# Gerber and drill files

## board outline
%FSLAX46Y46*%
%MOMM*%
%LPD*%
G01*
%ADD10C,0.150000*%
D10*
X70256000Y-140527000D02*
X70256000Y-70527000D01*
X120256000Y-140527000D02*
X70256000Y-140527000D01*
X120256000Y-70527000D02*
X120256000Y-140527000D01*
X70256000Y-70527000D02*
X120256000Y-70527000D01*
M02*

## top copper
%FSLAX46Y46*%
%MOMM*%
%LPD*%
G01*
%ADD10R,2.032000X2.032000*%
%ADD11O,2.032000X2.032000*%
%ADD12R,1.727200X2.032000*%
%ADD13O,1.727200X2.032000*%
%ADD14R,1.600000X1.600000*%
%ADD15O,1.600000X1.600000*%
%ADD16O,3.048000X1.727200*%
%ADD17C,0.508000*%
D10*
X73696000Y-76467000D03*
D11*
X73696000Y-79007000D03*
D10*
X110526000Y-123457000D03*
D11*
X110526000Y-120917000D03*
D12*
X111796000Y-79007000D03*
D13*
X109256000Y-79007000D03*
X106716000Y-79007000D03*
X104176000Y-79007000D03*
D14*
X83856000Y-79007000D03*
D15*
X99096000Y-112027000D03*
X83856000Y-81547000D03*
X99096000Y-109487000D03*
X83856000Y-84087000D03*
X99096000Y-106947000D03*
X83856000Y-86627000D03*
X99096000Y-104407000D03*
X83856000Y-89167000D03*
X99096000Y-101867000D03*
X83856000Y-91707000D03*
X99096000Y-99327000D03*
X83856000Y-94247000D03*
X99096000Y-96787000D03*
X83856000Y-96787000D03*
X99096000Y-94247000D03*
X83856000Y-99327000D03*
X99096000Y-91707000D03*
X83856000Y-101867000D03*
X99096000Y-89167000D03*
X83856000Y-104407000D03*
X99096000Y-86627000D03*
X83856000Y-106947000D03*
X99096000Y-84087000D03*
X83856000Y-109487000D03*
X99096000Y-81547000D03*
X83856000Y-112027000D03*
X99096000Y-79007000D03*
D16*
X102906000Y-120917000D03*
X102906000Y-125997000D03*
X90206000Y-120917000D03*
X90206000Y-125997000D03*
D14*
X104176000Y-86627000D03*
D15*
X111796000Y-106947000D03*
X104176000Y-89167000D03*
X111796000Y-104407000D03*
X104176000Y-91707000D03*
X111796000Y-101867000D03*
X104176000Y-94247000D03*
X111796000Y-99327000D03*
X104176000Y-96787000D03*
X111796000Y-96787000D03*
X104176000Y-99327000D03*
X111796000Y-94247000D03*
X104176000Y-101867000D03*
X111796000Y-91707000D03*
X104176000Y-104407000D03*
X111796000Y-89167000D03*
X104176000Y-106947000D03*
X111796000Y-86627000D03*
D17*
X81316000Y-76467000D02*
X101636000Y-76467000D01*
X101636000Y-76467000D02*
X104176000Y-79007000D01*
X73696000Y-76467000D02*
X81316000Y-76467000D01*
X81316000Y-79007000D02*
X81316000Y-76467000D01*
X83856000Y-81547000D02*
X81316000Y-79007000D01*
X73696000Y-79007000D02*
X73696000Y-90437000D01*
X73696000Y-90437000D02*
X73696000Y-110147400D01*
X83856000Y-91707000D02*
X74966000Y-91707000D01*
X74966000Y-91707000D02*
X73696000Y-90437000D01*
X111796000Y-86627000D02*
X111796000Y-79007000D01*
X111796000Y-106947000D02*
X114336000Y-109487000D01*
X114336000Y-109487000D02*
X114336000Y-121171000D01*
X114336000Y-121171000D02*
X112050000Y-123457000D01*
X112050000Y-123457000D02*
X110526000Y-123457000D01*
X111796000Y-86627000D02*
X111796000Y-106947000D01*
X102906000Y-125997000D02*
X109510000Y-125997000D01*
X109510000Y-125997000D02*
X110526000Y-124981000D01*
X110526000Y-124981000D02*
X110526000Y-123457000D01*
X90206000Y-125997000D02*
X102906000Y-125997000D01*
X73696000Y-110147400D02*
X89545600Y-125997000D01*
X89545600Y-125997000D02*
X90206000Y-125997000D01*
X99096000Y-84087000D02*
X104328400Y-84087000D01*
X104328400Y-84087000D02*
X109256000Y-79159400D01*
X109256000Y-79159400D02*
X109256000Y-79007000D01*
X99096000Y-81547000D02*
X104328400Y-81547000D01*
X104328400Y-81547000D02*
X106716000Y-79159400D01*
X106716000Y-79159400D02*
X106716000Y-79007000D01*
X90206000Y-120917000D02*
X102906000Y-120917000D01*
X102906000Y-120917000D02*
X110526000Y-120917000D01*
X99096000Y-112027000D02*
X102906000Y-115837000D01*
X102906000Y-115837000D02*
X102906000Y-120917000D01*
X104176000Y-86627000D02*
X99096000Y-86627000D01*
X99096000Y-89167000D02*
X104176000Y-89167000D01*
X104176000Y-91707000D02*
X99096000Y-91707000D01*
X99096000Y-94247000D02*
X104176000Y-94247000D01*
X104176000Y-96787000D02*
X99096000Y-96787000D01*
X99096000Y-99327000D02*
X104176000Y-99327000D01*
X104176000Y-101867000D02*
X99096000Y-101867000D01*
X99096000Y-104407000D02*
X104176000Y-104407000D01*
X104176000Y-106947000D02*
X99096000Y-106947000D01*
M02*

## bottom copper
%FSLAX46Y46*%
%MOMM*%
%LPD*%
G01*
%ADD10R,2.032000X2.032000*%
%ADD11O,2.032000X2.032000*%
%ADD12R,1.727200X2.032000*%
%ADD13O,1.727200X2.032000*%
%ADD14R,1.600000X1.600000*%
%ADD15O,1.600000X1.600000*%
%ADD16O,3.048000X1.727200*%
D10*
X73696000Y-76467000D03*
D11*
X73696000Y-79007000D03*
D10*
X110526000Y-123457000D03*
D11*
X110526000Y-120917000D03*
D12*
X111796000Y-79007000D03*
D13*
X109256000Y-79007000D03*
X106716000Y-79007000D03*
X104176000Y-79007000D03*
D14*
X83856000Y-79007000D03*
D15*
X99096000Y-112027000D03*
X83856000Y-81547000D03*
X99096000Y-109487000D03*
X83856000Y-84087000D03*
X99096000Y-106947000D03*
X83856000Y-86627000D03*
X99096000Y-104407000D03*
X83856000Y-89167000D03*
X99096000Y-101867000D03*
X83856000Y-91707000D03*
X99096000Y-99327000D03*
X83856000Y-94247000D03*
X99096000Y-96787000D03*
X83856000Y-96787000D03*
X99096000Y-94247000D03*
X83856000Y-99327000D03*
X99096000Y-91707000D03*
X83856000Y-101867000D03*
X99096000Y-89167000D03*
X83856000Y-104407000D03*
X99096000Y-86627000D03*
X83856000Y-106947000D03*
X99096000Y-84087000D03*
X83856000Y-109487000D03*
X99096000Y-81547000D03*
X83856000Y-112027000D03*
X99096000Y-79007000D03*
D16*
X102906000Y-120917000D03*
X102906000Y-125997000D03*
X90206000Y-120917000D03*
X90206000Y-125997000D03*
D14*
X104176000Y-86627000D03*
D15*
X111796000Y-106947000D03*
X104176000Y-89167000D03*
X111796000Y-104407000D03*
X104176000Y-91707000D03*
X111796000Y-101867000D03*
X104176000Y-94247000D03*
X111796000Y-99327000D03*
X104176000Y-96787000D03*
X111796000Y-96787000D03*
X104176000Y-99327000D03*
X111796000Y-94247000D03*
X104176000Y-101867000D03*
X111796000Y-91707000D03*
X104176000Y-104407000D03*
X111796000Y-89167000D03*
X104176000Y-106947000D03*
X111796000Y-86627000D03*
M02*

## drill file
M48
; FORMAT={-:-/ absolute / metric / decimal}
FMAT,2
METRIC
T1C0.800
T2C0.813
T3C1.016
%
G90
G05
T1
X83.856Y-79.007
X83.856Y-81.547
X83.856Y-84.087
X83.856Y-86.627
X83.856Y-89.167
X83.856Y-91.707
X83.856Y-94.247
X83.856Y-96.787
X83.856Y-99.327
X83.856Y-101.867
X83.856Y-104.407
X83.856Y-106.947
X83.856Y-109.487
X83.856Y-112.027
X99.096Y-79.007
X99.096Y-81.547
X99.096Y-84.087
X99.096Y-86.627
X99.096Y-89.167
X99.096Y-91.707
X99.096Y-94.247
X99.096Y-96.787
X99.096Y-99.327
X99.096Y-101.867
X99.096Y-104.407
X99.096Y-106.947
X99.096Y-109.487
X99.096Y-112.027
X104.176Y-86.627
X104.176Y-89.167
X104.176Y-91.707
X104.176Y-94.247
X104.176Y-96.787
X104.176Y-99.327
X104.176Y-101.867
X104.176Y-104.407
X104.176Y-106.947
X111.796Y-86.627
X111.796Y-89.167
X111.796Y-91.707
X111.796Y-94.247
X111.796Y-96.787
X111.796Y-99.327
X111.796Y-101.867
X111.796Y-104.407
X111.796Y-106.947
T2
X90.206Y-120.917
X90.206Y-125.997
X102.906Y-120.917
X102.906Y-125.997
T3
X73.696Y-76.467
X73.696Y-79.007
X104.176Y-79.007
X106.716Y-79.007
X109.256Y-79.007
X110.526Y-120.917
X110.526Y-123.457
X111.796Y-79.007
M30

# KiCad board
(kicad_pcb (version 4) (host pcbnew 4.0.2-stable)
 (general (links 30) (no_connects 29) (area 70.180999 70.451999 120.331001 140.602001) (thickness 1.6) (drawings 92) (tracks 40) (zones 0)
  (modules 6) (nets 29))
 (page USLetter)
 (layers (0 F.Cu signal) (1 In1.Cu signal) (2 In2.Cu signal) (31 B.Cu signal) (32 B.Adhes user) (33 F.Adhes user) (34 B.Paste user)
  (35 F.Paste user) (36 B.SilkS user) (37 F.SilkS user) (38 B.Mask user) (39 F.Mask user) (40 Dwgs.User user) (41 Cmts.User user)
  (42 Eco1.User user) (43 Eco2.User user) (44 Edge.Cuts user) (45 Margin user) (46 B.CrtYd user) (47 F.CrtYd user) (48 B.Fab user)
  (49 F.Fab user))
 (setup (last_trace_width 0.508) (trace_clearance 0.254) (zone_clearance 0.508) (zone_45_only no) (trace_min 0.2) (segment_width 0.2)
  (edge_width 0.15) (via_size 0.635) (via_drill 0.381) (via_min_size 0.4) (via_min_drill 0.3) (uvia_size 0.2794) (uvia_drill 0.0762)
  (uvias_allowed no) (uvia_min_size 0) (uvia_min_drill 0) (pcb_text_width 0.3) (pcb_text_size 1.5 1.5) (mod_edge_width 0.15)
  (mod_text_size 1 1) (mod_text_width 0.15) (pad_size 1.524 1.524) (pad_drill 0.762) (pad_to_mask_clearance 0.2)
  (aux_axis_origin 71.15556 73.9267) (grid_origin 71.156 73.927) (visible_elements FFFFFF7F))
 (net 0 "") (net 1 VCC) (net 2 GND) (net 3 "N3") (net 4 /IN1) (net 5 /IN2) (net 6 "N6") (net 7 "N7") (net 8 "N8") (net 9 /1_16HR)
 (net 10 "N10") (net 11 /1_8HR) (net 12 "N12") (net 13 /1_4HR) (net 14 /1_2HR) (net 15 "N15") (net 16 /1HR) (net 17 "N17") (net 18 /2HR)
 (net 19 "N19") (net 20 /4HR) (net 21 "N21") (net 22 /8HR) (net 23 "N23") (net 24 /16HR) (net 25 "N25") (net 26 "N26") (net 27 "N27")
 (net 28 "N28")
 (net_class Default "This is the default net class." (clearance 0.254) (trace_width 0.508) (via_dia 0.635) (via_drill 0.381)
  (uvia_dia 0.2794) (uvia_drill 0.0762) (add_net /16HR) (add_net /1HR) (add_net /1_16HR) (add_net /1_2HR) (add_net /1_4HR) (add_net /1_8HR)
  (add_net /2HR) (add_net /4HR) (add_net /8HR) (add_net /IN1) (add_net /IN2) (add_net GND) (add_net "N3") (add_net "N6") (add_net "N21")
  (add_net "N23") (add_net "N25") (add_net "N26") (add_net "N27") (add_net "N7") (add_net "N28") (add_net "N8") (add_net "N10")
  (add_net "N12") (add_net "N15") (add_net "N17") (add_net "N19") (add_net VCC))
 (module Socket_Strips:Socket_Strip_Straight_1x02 (layer F.Cu) (at 73.696 76.467 270)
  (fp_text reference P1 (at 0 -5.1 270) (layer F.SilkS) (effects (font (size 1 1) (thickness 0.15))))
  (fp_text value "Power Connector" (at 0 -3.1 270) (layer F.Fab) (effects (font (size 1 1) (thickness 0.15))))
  (pad 1 thru_hole rect (at 0 0 270) (size 2.032 2.032) (drill 1.016) (layers *.Cu *.Mask) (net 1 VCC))
  (pad 2 thru_hole oval (at 2.54 0 270) (size 2.032 2.032) (drill 1.016) (layers *.Cu *.Mask) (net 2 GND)))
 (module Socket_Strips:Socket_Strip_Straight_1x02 (layer F.Cu) (at 110.526 123.457 90)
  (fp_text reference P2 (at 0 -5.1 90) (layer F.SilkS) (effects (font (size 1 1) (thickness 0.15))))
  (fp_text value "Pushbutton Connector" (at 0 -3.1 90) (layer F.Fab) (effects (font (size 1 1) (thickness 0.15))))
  (pad 1 thru_hole rect (at 0 0 90) (size 2.032 2.032) (drill 1.016) (layers *.Cu *.Mask) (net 2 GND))
  (pad 2 thru_hole oval (at 2.54 0 90) (size 2.032 2.032) (drill 1.016) (layers *.Cu *.Mask) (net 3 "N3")))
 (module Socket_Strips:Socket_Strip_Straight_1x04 (layer F.Cu) (at 111.796 79.007 180)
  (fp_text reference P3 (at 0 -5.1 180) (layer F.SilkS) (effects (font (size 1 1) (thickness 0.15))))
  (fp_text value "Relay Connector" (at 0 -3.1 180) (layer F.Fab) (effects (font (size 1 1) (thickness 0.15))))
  (pad 1 thru_hole rect (at 0 0 180) (size 1.7272 2.032) (drill 1.016) (layers *.Cu *.Mask) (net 2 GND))
  (pad 2 thru_hole oval (at 2.54 0 180) (size 1.7272 2.032) (drill 1.016) (layers *.Cu *.Mask) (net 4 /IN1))
  (pad 3 thru_hole oval (at 5.08 0 180) (size 1.7272 2.032) (drill 1.016) (layers *.Cu *.Mask) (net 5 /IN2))
  (pad 4 thru_hole oval (at 7.62 0 180) (size 1.7272 2.032) (drill 1.016) (layers *.Cu *.Mask) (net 1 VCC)))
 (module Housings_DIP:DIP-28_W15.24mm (layer F.Cu) (at 83.856 79.007)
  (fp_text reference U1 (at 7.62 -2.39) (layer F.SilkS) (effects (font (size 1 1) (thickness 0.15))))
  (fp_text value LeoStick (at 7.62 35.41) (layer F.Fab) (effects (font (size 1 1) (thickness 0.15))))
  (pad 1 thru_hole rect (at 0 0) (size 1.6 1.6) (drill 0.8) (layers *.Cu *.Mask) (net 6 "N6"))
  (pad 15 thru_hole oval (at 15.24 33.02) (size 1.6 1.6) (drill 0.8) (layers *.Cu *.Mask) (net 3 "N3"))
  (pad 2 thru_hole oval (at 0 2.54) (size 1.6 1.6) (drill 0.8) (layers *.Cu *.Mask) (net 1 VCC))
  (pad 16 thru_hole oval (at 15.24 30.48) (size 1.6 1.6) (drill 0.8) (layers *.Cu *.Mask) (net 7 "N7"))
  (pad 3 thru_hole oval (at 0 5.08) (size 1.6 1.6) (drill 0.8) (layers *.Cu *.Mask) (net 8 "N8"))
  (pad 17 thru_hole oval (at 15.24 27.94) (size 1.6 1.6) (drill 0.8) (layers *.Cu *.Mask) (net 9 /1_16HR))
  (pad 4 thru_hole oval (at 0 7.62) (size 1.6 1.6) (drill 0.8) (layers *.Cu *.Mask) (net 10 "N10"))
  (pad 18 thru_hole oval (at 15.24 25.4) (size 1.6 1.6) (drill 0.8) (layers *.Cu *.Mask) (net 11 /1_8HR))
  (pad 5 thru_hole oval (at 0 10.16) (size 1.6 1.6) (drill 0.8) (layers *.Cu *.Mask) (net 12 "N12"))
  (pad 19 thru_hole oval (at 15.24 22.86) (size 1.6 1.6) (drill 0.8) (layers *.Cu *.Mask) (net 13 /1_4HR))
  (pad 6 thru_hole oval (at 0 12.7) (size 1.6 1.6) (drill 0.8) (layers *.Cu *.Mask) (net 2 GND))
  (pad 20 thru_hole oval (at 15.24 20.32) (size 1.6 1.6) (drill 0.8) (layers *.Cu *.Mask) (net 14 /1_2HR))
  (pad 7 thru_hole oval (at 0 15.24) (size 1.6 1.6) (drill 0.8) (layers *.Cu *.Mask) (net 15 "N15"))
  (pad 21 thru_hole oval (at 15.24 17.78) (size 1.6 1.6) (drill 0.8) (layers *.Cu *.Mask) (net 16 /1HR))
  (pad 8 thru_hole oval (at 0 17.78) (size 1.6 1.6) (drill 0.8) (layers *.Cu *.Mask) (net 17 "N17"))
  (pad 22 thru_hole oval (at 15.24 15.24) (size 1.6 1.6) (drill 0.8) (layers *.Cu *.Mask) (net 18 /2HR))
  (pad 9 thru_hole oval (at 0 20.32) (size 1.6 1.6) (drill 0.8) (layers *.Cu *.Mask) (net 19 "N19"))
  (pad 23 thru_hole oval (at 15.24 12.7) (size 1.6 1.6) (drill 0.8) (layers *.Cu *.Mask) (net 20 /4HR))
  (pad 10 thru_hole oval (at 0 22.86) (size 1.6 1.6) (drill 0.8) (layers *.Cu *.Mask) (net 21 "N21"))
  (pad 24 thru_hole oval (at 15.24 10.16) (size 1.6 1.6) (drill 0.8) (layers *.Cu *.Mask) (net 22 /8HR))
  (pad 11 thru_hole oval (at 0 25.4) (size 1.6 1.6) (drill 0.8) (layers *.Cu *.Mask) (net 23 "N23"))
  (pad 25 thru_hole oval (at 15.24 7.62) (size 1.6 1.6) (drill 0.8) (layers *.Cu *.Mask) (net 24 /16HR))
  (pad 12 thru_hole oval (at 0 27.94) (size 1.6 1.6) (drill 0.8) (layers *.Cu *.Mask) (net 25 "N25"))
  (pad 26 thru_hole oval (at 15.24 5.08) (size 1.6 1.6) (drill 0.8) (layers *.Cu *.Mask) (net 4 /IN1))
  (pad 13 thru_hole oval (at 0 30.48) (size 1.6 1.6) (drill 0.8) (layers *.Cu *.Mask) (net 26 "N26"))
  (pad 27 thru_hole oval (at 15.24 2.54) (size 1.6 1.6) (drill 0.8) (layers *.Cu *.Mask) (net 5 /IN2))
  (pad 14 thru_hole oval (at 0 33.02) (size 1.6 1.6) (drill 0.8) (layers *.Cu *.Mask) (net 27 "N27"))
  (pad 28 thru_hole oval (at 15.24 0) (size 1.6 1.6) (drill 0.8) (layers *.Cu *.Mask) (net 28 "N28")))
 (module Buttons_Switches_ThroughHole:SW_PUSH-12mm (layer F.Cu) (at 96.556 123.457)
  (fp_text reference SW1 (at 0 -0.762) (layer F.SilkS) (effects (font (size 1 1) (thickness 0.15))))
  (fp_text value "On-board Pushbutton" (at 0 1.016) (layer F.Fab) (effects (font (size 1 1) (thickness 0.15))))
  (pad 1 thru_hole oval (at 6.35 -2.54) (size 3.048 1.7272) (drill 0.8128) (layers *.Cu *.Mask) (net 3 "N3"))
  (pad 2 thru_hole oval (at 6.35 2.54) (size 3.048 1.7272) (drill 0.8128) (layers *.Cu *.Mask) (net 2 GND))
  (pad 1 thru_hole oval (at -6.35 -2.54) (size 3.048 1.7272) (drill 0.8128) (layers *.Cu *.Mask) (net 3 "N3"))
  (pad 2 thru_hole oval (at -6.35 2.54) (size 3.048 1.7272) (drill 0.8128) (layers *.Cu *.Mask) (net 2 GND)))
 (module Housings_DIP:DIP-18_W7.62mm (layer F.Cu) (at 104.176 86.627)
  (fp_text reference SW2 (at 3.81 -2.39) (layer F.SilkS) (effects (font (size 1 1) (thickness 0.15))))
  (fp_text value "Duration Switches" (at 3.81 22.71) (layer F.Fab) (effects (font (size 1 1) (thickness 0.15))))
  (pad 1 thru_hole rect (at 0 0) (size 1.6 1.6) (drill 0.8) (layers *.Cu *.Mask) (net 24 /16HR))
  (pad 10 thru_hole oval (at 7.62 20.32) (size 1.6 1.6) (drill 0.8) (layers *.Cu *.Mask) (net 2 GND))
  (pad 2 thru_hole oval (at 0 2.54) (size 1.6 1.6) (drill 0.8) (layers *.Cu *.Mask) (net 22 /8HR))
  (pad 11 thru_hole oval (at 7.62 17.78) (size 1.6 1.6) (drill 0.8) (layers *.Cu *.Mask) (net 2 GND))
  (pad 3 thru_hole oval (at 0 5.08) (size 1.6 1.6) (drill 0.8) (layers *.Cu *.Mask) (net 20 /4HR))
  (pad 12 thru_hole oval (at 7.62 15.24) (size 1.6 1.6) (drill 0.8) (layers *.Cu *.Mask) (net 2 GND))
  (pad 4 thru_hole oval (at 0 7.62) (size 1.6 1.6) (drill 0.8) (layers *.Cu *.Mask) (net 18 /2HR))
  (pad 13 thru_hole oval (at 7.62 12.7) (size 1.6 1.6) (drill 0.8) (layers *.Cu *.Mask) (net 2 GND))
  (pad 5 thru_hole oval (at 0 10.16) (size 1.6 1.6) (drill 0.8) (layers *.Cu *.Mask) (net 16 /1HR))
  (pad 14 thru_hole oval (at 7.62 10.16) (size 1.6 1.6) (drill 0.8) (layers *.Cu *.Mask) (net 2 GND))
  (pad 6 thru_hole oval (at 0 12.7) (size 1.6 1.6) (drill 0.8) (layers *.Cu *.Mask) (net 14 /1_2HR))
  (pad 15 thru_hole oval (at 7.62 7.62) (size 1.6 1.6) (drill 0.8) (layers *.Cu *.Mask) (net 2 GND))
  (pad 7 thru_hole oval (at 0 15.24) (size 1.6 1.6) (drill 0.8) (layers *.Cu *.Mask) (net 13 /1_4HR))
  (pad 16 thru_hole oval (at 7.62 5.08) (size 1.6 1.6) (drill 0.8) (layers *.Cu *.Mask) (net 2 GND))
  (pad 8 thru_hole oval (at 0 17.78) (size 1.6 1.6) (drill 0.8) (layers *.Cu *.Mask) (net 11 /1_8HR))
  (pad 17 thru_hole oval (at 7.62 2.54) (size 1.6 1.6) (drill 0.8) (layers *.Cu *.Mask) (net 2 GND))
  (pad 9 thru_hole oval (at 0 20.32) (size 1.6 1.6) (drill 0.8) (layers *.Cu *.Mask) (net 9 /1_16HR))
  (pad 18 thru_hole oval (at 7.62 0) (size 1.6 1.6) (drill 0.8) (layers *.Cu *.Mask) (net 2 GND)))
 (gr_line (start 70.256 140.527) (end 70.256 70.527) (angle 90) (layer Edge.Cuts) (width 0.15))
 (gr_line (start 120.256 140.527) (end 70.256 140.527) (angle 90) (layer Edge.Cuts) (width 0.15))
 (gr_line (start 120.256 70.527) (end 120.256 140.527) (angle 90) (layer Edge.Cuts) (width 0.15))
 (gr_line (start 70.256 70.527) (end 120.256 70.527) (angle 90) (layer Edge.Cuts) (width 0.15))
 (segment (start 81.316 76.467) (end 101.636 76.467) (width 0.508) (layer F.Cu) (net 1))
 (segment (start 101.636 76.467) (end 104.176 79.007) (width 0.508) (layer F.Cu) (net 1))
 (segment (start 73.696 76.467) (end 81.316 76.467) (width 0.508) (layer F.Cu) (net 1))
 (segment (start 81.316 79.007) (end 81.316 76.467) (width 0.508) (layer F.Cu) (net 1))
 (segment (start 83.856 81.547) (end 81.316 79.007) (width 0.508) (layer F.Cu) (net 1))
 (segment (start 73.696 79.007) (end 73.696 90.437) (width 0.508) (layer F.Cu) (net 2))
 (segment (start 73.696 90.437) (end 73.696 110.1474) (width 0.508) (layer F.Cu) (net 2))
 (segment (start 83.856 91.707) (end 74.966 91.707) (width 0.508) (layer F.Cu) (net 2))
 (segment (start 74.966 91.707) (end 73.696 90.437) (width 0.508) (layer F.Cu) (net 2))
 (segment (start 111.796 86.627) (end 111.796 79.007) (width 0.508) (layer F.Cu) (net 2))
 (segment (start 111.796 106.947) (end 114.336 109.487) (width 0.508) (layer F.Cu) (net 2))
 (segment (start 114.336 109.487) (end 114.336 121.171) (width 0.508) (layer F.Cu) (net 2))
 (segment (start 114.336 121.171) (end 112.05 123.457) (width 0.508) (layer F.Cu) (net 2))
 (segment (start 112.05 123.457) (end 110.526 123.457) (width 0.508) (layer F.Cu) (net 2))
 (segment (start 111.796 86.627) (end 111.796 106.947) (width 0.508) (layer F.Cu) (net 2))
 (segment (start 102.906 125.997) (end 109.51 125.997) (width 0.508) (layer F.Cu) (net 2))
 (segment (start 109.51 125.997) (end 110.526 124.981) (width 0.508) (layer F.Cu) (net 2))
 (segment (start 110.526 124.981) (end 110.526 123.457) (width 0.508) (layer F.Cu) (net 2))
 (segment (start 90.206 125.997) (end 102.906 125.997) (width 0.508) (layer F.Cu) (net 2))
 (segment (start 73.696 110.1474) (end 89.5456 125.997) (width 0.508) (layer F.Cu) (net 2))
 (segment (start 89.5456 125.997) (end 90.206 125.997) (width 0.508) (layer F.Cu) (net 2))
 (segment (start 99.096 84.087) (end 104.3284 84.087) (width 0.508) (layer F.Cu) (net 4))
 (segment (start 104.3284 84.087) (end 109.256 79.1594) (width 0.508) (layer F.Cu) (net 4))
 (segment (start 109.256 79.1594) (end 109.256 79.007) (width 0.508) (layer F.Cu) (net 4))
 (segment (start 99.096 81.547) (end 104.3284 81.547) (width 0.508) (layer F.Cu) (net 5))
 (segment (start 104.3284 81.547) (end 106.716 79.1594) (width 0.508) (layer F.Cu) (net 5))
 (segment (start 106.716 79.1594) (end 106.716 79.007) (width 0.508) (layer F.Cu) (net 5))
 (segment (start 90.206 120.917) (end 102.906 120.917) (width 0.508) (layer F.Cu) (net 3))
 (segment (start 102.906 120.917) (end 110.526 120.917) (width 0.508) (layer F.Cu) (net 3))
 (segment (start 99.096 112.027) (end 102.906 115.837) (width 0.508) (layer F.Cu) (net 3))
 (segment (start 102.906 115.837) (end 102.906 120.917) (width 0.508) (layer F.Cu) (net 3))
 (segment (start 104.176 86.627) (end 99.096 86.627) (width 0.508) (layer F.Cu) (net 24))
 (segment (start 99.096 89.167) (end 104.176 89.167) (width 0.508) (layer F.Cu) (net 22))
 (segment (start 104.176 91.707) (end 99.096 91.707) (width 0.508) (layer F.Cu) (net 20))
 (segment (start 99.096 94.247) (end 104.176 94.247) (width 0.508) (layer F.Cu) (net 18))
 (segment (start 104.176 96.787) (end 99.096 96.787) (width 0.508) (layer F.Cu) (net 16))
 (segment (start 99.096 99.327) (end 104.176 99.327) (width 0.508) (layer F.Cu) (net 14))
 (segment (start 104.176 101.867) (end 99.096 101.867) (width 0.508) (layer F.Cu) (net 13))
 (segment (start 99.096 104.407) (end 104.176 104.407) (width 0.508) (layer F.Cu) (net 11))
 (segment (start 104.176 106.947) (end 99.096 106.947) (width 0.508) (layer F.Cu) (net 9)))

